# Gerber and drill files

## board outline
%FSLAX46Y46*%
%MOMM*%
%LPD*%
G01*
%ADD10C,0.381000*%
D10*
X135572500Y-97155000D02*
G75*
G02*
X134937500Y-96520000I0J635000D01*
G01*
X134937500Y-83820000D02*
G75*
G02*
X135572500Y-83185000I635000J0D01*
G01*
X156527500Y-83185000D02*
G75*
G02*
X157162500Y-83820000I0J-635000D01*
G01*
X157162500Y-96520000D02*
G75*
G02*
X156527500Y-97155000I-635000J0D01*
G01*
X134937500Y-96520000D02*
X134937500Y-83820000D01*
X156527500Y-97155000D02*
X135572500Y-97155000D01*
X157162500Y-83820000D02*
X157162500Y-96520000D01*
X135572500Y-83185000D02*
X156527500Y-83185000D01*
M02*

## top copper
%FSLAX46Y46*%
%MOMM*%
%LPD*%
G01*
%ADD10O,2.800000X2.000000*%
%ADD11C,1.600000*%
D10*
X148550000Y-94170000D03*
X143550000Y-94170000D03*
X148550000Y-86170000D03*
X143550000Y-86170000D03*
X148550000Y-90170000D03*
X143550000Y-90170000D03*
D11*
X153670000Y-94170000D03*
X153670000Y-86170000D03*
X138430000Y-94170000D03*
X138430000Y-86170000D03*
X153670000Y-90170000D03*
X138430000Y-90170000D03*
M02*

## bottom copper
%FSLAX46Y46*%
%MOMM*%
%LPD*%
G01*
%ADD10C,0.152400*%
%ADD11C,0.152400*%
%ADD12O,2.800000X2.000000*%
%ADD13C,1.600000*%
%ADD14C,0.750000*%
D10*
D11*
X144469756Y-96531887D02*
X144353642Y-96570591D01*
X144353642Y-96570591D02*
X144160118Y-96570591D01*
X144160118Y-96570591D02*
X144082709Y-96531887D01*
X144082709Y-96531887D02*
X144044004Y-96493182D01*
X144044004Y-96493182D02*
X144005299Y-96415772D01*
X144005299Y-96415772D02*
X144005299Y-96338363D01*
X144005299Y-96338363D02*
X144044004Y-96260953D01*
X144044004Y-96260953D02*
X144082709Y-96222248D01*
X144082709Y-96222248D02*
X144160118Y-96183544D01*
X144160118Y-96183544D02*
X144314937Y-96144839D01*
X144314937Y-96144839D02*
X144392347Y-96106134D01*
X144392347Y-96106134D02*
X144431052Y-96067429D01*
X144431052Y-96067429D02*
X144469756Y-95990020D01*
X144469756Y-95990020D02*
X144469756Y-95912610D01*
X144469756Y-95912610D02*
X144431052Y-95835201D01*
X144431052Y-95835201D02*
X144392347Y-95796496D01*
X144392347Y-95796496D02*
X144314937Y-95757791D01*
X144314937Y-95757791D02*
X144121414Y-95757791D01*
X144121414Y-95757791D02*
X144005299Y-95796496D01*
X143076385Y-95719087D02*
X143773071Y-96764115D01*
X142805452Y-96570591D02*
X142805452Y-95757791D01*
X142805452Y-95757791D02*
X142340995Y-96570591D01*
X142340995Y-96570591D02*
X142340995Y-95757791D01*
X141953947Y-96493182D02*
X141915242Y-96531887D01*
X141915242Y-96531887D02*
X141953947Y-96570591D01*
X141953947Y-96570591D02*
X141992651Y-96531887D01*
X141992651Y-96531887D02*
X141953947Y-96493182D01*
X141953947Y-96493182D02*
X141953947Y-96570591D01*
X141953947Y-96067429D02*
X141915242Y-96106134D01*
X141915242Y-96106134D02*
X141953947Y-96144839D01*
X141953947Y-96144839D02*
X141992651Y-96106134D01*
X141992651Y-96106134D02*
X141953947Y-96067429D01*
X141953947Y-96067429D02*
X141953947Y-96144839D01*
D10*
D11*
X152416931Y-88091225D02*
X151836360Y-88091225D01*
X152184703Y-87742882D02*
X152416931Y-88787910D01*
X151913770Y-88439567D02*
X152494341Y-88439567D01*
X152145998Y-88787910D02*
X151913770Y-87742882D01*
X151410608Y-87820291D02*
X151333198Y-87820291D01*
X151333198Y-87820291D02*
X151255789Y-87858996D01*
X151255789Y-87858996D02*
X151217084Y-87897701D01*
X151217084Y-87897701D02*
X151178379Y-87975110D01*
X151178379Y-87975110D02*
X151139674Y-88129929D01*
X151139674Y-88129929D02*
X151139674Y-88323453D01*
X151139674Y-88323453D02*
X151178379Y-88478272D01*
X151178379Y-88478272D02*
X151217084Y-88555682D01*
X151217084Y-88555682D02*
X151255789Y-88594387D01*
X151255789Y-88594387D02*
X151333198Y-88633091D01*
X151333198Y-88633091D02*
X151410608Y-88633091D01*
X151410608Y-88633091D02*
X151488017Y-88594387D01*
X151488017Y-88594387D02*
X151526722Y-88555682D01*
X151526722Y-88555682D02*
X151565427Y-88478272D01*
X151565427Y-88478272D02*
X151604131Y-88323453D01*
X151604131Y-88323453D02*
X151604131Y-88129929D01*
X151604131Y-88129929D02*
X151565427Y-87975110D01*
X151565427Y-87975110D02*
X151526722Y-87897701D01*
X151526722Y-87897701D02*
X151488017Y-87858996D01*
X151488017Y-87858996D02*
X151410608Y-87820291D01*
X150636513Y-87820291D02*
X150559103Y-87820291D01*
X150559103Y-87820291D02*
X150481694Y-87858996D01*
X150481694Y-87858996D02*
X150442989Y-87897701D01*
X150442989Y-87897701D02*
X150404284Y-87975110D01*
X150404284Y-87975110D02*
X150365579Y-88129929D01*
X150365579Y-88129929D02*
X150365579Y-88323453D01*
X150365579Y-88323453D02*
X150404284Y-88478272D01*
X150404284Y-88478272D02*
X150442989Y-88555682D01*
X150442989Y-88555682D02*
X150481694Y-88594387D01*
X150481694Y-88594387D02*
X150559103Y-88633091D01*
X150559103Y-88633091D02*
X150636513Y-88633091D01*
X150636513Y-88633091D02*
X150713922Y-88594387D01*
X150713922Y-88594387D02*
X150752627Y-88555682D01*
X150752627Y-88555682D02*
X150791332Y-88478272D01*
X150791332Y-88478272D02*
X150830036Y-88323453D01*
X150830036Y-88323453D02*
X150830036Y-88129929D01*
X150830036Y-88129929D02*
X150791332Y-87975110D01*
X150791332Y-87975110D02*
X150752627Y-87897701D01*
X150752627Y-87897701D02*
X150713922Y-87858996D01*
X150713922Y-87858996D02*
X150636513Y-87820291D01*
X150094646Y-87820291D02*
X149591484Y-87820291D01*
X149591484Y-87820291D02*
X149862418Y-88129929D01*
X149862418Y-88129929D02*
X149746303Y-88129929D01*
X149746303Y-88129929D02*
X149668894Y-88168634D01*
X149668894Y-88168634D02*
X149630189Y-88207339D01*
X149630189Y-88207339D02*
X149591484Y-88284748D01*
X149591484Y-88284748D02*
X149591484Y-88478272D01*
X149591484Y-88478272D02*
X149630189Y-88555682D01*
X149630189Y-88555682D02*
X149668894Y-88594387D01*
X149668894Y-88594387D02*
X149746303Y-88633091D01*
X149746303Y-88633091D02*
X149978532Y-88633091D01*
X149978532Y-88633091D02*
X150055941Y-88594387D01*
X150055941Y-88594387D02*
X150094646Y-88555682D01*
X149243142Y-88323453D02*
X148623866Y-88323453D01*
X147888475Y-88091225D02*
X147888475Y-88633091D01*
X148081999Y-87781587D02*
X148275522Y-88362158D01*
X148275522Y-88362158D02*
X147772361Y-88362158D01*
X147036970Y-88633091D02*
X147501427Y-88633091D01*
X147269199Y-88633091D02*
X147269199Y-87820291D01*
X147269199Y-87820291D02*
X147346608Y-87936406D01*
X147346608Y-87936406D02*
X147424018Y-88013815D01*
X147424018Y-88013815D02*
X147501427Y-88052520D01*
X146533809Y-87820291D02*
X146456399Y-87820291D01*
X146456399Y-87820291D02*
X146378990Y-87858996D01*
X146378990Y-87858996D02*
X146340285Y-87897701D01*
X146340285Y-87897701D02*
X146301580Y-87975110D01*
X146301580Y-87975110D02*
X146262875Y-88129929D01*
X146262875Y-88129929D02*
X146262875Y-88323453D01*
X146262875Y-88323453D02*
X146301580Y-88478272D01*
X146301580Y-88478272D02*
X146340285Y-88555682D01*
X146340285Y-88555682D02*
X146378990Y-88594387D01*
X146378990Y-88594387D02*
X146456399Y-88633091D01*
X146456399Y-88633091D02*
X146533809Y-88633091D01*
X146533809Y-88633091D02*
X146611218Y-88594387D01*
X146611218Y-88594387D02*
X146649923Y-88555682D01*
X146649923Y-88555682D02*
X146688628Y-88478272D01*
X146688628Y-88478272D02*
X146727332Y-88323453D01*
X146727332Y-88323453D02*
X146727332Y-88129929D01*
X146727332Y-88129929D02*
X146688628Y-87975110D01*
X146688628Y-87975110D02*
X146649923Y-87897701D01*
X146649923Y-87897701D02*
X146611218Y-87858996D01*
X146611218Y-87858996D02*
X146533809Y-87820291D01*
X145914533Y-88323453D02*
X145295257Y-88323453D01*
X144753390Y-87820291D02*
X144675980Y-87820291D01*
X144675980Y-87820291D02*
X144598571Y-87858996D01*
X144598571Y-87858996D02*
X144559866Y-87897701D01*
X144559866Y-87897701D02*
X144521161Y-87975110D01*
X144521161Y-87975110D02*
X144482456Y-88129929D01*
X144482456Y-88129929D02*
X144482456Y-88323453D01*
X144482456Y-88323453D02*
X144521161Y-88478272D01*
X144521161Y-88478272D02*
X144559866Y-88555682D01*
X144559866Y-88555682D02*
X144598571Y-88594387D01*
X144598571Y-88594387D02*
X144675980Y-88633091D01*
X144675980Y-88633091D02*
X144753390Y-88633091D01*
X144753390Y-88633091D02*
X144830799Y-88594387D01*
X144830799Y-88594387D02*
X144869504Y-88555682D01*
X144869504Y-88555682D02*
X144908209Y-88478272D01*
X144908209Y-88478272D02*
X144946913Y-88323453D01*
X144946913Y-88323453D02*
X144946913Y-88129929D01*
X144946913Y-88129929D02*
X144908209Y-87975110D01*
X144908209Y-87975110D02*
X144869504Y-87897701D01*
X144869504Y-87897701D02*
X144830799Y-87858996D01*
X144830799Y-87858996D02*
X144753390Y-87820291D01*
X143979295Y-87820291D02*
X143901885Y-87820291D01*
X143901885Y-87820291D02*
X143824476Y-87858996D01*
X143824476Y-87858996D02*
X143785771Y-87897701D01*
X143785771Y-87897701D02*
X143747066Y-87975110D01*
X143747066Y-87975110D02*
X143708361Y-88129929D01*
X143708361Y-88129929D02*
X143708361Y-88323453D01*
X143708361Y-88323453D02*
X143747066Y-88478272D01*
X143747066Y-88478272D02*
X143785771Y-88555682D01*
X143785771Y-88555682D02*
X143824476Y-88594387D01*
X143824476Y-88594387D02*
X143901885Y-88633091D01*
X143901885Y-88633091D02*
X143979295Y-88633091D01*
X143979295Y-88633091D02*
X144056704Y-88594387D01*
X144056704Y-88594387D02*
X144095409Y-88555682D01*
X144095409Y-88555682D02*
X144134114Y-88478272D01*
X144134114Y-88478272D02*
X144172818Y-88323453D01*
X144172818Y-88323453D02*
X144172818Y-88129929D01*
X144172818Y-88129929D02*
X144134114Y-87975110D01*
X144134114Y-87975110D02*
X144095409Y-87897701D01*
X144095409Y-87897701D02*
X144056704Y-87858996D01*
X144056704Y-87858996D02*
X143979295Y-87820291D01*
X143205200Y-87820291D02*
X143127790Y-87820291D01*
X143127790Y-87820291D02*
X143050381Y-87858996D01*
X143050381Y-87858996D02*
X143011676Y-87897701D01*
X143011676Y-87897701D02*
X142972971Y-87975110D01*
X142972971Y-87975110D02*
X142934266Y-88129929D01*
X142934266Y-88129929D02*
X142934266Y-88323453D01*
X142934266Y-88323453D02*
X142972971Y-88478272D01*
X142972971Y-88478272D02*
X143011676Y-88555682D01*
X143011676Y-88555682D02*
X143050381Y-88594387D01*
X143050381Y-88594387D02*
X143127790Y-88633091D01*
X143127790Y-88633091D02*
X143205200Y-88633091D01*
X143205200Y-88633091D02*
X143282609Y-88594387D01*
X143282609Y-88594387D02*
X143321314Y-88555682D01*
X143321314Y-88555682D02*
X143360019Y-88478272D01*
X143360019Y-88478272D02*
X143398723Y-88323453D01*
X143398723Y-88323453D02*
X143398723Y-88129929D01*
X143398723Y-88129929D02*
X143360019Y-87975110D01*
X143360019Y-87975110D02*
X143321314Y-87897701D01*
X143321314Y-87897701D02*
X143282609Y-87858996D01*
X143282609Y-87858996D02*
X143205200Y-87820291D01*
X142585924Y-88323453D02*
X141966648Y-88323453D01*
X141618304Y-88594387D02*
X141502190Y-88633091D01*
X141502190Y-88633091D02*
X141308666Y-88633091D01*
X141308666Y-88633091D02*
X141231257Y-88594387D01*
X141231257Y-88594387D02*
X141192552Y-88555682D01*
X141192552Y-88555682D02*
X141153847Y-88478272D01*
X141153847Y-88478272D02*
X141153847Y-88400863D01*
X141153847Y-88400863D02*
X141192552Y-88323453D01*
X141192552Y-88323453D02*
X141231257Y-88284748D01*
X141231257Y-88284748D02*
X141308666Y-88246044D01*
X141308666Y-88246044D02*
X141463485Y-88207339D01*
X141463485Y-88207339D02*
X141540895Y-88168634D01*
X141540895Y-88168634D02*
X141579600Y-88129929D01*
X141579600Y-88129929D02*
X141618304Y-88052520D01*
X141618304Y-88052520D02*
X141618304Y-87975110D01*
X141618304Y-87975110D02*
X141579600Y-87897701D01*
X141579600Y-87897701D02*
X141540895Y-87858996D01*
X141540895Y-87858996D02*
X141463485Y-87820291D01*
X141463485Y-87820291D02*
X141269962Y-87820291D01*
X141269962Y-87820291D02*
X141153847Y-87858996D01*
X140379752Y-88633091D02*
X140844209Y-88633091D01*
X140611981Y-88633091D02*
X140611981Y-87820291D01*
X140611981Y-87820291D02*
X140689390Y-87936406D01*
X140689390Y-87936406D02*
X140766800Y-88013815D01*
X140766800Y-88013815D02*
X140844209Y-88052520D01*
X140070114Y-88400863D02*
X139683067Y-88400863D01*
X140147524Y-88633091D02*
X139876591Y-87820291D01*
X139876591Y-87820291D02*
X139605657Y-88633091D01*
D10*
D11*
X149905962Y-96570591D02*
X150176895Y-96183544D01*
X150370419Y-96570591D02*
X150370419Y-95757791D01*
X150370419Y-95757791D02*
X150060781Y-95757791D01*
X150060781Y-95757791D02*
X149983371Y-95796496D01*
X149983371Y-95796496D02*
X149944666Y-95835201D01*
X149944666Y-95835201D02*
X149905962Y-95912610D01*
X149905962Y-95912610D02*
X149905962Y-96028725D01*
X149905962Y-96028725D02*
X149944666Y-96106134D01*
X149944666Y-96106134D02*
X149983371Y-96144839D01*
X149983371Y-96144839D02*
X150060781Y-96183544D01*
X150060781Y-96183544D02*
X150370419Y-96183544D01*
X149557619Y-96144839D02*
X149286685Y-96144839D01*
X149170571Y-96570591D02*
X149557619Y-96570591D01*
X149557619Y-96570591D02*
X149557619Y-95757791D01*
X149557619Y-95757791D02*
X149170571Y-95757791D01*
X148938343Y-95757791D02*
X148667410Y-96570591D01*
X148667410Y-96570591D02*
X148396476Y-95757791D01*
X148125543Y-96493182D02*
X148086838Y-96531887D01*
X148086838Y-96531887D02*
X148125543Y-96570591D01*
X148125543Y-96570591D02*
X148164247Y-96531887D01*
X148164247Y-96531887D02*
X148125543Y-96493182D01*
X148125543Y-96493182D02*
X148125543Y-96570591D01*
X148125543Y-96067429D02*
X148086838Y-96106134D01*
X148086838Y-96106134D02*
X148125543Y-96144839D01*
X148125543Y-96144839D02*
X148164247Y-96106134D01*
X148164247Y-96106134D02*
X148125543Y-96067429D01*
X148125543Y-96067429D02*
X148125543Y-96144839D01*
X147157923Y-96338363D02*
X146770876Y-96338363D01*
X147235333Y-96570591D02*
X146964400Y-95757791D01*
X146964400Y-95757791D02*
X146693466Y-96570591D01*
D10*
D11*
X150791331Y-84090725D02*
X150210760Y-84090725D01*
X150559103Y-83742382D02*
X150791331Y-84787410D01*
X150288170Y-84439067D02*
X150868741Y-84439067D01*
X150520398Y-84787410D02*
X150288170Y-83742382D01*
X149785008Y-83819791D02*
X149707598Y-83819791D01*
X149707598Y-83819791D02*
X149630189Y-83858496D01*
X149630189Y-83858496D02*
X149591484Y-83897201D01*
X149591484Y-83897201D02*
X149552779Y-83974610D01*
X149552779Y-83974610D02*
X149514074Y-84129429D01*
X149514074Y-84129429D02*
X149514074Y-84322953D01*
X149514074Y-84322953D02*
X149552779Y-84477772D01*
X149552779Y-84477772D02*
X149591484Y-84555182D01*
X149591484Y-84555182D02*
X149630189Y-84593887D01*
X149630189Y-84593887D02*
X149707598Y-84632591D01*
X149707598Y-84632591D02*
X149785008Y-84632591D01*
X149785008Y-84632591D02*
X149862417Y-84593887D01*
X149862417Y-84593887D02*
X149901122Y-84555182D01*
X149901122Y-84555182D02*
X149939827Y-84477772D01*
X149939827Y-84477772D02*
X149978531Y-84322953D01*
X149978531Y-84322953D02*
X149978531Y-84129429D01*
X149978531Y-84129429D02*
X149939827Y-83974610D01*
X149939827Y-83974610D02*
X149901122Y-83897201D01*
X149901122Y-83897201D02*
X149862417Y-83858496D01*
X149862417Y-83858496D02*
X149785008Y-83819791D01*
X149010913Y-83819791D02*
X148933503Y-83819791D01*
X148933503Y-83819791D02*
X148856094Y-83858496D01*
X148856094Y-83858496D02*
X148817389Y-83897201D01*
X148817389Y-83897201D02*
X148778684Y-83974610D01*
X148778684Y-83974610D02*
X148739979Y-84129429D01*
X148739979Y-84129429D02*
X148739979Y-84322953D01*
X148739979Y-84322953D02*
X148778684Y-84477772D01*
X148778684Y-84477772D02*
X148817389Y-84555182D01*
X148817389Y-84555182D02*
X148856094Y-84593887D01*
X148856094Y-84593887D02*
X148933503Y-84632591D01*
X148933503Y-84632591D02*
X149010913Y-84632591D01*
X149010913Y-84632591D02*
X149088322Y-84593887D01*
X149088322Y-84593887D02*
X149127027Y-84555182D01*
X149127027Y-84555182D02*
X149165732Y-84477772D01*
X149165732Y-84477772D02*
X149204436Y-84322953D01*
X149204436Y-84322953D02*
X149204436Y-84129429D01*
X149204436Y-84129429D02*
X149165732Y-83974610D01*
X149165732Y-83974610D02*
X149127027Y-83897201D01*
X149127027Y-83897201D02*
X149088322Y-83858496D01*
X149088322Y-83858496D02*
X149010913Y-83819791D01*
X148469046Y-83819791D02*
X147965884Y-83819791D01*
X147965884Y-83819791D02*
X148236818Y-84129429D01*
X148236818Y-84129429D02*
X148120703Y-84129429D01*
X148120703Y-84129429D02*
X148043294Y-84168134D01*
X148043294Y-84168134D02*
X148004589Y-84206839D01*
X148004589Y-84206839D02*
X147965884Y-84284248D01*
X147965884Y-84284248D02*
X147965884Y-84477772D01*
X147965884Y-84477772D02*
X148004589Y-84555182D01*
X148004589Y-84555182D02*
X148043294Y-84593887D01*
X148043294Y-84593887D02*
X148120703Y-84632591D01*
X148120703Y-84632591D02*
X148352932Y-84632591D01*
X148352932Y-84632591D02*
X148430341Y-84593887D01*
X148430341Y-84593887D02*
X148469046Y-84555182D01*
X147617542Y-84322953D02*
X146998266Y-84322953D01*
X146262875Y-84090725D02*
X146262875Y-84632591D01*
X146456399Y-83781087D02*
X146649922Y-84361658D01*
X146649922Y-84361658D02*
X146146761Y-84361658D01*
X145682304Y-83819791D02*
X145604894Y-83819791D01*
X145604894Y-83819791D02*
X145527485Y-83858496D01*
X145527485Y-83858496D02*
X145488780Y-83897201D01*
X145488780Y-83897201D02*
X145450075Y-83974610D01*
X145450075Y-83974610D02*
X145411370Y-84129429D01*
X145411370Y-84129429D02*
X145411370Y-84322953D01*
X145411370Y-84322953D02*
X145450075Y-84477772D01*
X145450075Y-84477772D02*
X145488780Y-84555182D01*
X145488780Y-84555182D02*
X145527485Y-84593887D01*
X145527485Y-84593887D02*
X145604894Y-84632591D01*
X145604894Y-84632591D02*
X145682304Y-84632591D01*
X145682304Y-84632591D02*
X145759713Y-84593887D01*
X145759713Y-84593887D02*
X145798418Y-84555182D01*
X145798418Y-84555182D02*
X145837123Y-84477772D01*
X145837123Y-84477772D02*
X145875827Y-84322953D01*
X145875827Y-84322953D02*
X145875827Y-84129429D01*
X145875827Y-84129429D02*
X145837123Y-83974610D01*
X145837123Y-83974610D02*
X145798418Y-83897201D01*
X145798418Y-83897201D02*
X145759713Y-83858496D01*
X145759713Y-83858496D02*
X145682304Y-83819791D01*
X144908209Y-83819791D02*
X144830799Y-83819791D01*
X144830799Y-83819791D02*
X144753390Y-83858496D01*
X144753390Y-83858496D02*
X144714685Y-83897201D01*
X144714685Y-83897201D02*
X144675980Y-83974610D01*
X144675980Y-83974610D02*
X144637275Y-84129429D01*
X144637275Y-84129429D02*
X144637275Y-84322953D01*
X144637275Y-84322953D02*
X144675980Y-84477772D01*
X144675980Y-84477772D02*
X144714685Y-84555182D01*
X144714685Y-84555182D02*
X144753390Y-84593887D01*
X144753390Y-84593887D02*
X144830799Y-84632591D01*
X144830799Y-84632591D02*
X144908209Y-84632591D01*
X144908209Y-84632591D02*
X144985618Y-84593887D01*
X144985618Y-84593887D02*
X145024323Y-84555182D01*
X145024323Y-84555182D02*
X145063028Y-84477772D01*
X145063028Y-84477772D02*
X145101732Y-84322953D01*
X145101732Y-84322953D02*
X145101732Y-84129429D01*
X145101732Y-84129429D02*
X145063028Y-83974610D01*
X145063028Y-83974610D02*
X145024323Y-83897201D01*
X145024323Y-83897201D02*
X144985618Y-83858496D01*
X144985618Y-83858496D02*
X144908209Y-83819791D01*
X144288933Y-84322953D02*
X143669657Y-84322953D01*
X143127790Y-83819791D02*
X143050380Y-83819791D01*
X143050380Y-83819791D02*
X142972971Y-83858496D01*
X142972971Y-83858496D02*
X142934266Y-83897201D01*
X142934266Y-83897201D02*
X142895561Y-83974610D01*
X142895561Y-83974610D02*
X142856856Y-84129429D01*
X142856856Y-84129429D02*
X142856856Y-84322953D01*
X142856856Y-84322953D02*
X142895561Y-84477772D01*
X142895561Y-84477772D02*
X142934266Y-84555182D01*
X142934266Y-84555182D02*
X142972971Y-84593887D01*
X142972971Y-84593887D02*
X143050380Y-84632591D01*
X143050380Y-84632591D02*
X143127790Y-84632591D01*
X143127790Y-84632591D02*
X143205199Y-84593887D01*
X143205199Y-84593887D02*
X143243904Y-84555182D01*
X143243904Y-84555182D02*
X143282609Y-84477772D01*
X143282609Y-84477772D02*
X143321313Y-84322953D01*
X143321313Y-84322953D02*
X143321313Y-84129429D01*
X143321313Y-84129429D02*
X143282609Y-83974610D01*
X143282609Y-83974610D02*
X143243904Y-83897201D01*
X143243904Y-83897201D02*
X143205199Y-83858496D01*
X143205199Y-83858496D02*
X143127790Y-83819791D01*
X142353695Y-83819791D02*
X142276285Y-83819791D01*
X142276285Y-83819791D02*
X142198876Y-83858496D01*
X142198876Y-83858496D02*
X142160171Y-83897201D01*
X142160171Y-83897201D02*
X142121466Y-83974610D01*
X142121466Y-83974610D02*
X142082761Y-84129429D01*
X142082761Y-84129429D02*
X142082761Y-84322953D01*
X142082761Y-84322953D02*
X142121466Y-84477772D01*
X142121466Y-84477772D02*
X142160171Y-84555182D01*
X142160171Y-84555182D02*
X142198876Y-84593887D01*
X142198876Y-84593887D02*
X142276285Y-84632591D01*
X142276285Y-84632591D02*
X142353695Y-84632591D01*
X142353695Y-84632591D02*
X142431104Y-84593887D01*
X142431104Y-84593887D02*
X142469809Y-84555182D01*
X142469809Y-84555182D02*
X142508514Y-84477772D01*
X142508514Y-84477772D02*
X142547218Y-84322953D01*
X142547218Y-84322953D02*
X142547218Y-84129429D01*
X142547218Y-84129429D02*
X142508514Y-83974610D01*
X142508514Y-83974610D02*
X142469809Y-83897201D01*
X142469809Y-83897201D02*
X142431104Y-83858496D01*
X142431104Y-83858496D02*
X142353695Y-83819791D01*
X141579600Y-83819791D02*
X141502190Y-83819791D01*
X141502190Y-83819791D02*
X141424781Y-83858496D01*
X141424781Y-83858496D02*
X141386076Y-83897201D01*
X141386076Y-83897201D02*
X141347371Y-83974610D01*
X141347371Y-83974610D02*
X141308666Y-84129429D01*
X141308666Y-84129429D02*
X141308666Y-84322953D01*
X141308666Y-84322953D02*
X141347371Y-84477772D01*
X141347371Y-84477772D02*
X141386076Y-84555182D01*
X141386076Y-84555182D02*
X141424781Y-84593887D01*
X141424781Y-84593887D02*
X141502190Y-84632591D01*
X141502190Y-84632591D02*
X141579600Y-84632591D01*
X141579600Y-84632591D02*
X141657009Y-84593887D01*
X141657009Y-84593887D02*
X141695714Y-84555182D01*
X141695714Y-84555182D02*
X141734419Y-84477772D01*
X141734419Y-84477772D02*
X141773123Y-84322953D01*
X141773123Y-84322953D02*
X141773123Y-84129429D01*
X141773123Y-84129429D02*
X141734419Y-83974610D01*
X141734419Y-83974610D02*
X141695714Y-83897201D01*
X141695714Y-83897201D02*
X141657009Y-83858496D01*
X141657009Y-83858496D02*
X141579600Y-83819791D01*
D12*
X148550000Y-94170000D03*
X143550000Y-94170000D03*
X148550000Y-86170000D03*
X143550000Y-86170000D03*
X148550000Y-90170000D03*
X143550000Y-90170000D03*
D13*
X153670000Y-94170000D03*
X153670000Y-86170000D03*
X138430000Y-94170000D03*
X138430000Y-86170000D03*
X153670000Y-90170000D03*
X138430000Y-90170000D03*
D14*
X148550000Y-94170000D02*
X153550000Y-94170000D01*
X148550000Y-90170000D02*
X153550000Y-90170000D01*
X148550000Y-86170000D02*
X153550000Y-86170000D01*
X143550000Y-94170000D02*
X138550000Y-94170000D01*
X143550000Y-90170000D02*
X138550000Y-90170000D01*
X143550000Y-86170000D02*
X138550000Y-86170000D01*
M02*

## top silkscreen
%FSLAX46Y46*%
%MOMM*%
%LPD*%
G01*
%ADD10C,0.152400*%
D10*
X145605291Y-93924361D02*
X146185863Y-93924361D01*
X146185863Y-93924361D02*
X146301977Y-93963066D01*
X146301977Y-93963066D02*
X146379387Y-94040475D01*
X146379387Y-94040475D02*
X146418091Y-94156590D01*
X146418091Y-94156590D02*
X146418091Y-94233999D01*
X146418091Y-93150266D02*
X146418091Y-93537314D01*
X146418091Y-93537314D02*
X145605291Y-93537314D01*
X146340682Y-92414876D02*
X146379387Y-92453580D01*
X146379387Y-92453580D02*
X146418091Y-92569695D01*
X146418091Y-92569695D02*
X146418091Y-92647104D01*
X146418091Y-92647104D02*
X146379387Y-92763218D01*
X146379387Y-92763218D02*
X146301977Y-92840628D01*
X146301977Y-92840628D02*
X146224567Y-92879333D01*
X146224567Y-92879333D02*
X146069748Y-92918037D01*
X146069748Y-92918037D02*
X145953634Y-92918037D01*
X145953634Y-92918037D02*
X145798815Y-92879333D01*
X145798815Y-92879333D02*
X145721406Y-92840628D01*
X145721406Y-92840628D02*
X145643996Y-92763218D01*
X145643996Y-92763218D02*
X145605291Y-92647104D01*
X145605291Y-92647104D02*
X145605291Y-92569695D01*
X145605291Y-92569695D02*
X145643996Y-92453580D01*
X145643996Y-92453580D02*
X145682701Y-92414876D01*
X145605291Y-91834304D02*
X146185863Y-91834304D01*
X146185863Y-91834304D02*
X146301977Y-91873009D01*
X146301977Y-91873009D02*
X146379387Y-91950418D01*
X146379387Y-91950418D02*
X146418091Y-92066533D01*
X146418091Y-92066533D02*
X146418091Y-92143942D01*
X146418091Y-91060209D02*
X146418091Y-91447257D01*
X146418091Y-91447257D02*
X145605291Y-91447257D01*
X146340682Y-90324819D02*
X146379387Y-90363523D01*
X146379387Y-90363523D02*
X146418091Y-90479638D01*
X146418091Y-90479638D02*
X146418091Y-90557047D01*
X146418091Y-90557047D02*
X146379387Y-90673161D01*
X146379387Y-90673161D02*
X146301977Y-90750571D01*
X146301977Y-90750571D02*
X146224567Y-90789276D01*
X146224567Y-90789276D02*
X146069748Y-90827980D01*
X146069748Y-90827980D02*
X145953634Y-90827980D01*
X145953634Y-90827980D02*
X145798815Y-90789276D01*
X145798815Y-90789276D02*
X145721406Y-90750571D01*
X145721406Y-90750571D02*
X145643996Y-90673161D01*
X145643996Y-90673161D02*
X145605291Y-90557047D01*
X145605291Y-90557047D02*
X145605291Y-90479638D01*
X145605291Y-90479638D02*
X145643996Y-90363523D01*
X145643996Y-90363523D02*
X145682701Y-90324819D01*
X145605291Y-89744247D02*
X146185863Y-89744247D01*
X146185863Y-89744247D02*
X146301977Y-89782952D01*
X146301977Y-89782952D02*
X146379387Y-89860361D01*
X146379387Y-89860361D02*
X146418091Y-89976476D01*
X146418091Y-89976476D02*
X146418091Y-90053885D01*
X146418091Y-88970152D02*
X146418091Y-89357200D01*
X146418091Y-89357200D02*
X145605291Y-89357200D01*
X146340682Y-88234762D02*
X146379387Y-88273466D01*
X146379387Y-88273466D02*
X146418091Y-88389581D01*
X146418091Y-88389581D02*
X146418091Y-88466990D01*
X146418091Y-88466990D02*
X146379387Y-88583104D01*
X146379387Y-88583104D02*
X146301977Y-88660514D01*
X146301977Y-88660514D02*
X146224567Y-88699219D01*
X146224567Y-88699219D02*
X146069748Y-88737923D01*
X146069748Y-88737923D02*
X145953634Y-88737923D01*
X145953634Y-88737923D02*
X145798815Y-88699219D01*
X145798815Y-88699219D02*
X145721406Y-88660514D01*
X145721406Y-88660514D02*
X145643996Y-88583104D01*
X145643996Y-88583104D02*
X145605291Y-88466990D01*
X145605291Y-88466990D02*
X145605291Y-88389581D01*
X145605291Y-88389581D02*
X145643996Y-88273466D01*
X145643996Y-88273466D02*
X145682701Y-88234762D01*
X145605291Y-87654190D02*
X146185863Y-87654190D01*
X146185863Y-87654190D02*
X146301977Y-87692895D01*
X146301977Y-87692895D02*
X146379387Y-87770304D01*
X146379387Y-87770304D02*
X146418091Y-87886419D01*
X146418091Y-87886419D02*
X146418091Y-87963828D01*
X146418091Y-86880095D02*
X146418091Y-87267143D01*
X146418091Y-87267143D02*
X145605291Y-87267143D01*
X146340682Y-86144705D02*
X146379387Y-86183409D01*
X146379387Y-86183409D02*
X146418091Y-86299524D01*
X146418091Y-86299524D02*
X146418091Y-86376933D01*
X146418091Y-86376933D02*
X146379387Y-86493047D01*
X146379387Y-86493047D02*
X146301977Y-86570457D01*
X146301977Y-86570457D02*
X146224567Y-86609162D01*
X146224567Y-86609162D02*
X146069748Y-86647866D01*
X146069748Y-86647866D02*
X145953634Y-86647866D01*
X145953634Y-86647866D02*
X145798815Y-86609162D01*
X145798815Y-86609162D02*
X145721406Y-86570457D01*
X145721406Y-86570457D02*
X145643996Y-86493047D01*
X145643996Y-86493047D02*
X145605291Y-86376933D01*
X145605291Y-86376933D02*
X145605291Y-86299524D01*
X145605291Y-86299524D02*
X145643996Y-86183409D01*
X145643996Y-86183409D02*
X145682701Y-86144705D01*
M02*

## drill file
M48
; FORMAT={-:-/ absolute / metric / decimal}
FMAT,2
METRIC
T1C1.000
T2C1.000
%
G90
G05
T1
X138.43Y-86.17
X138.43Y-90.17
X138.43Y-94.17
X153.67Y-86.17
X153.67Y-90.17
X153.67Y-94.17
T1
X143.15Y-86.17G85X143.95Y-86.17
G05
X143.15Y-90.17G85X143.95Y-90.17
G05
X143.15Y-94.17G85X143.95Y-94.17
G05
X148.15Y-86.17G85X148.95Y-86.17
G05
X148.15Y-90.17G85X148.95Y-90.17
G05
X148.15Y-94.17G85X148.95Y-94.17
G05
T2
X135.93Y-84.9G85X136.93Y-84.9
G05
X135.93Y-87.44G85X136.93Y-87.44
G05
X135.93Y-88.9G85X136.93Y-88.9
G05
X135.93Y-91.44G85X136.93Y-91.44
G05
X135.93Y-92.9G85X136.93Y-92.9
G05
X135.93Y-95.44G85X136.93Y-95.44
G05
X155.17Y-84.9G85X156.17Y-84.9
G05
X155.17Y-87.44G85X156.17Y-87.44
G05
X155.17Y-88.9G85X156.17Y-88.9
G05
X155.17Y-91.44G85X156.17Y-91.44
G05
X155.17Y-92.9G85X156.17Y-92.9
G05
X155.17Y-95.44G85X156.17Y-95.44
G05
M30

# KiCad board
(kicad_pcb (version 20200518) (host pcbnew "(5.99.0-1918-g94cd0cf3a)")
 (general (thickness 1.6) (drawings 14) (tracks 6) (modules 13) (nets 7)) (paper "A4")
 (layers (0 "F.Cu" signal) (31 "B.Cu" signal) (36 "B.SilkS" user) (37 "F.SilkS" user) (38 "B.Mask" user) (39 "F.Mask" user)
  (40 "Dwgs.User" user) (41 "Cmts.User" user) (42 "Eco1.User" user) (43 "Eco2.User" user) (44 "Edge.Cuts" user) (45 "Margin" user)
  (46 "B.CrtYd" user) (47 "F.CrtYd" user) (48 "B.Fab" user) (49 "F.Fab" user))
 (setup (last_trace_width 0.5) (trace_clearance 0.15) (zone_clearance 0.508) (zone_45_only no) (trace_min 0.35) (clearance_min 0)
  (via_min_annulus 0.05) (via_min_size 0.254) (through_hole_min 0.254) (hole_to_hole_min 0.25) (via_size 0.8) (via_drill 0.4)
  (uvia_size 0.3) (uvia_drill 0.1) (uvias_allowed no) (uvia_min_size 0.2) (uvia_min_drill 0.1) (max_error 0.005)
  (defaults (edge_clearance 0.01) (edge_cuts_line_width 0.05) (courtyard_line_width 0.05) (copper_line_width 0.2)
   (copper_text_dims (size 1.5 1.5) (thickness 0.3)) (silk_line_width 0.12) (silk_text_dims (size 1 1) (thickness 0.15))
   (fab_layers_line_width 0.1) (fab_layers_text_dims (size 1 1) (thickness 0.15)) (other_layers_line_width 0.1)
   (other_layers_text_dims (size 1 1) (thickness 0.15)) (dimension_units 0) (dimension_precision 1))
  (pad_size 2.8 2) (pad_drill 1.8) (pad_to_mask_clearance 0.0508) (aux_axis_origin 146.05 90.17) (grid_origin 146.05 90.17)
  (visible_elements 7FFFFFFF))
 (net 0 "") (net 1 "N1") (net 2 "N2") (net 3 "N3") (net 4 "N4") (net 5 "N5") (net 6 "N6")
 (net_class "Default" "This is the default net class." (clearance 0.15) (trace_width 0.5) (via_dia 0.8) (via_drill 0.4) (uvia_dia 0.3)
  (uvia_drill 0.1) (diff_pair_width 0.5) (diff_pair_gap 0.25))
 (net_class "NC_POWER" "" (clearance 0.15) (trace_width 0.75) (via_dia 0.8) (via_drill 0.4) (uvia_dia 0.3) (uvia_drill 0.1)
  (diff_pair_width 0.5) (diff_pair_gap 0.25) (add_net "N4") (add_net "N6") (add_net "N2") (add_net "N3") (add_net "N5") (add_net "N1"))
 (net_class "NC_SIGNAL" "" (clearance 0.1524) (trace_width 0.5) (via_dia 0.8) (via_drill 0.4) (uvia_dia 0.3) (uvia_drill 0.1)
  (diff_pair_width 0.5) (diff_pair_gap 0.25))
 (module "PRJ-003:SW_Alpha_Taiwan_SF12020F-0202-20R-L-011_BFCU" (layer "F.Cu") (at 146.05 90.17)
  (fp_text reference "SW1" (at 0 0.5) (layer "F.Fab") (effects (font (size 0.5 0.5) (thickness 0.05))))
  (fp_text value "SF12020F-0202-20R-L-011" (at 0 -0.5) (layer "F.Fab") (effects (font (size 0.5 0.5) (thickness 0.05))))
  (pad "" connect oval (at 2.5 4) (size 1.8 1) (layers "F.Mask"))
  (pad "6" thru_hole oval (at 2.5 4) (size 2.8 2) (drill oval 1.8 1) (layers *.Cu *.Mask) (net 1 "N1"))
  (pad "3" thru_hole oval (at -2.5 4) (size 2.8 2) (drill oval 1.8 1) (layers *.Cu *.Mask) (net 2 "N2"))
  (pad "4" thru_hole oval (at 2.5 -4) (size 2.8 2) (drill oval 1.8 1) (layers *.Cu *.Mask) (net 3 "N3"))
  (pad "1" thru_hole oval (at -2.5 -4) (size 2.8 2) (drill oval 1.8 1) (layers *.Cu *.Mask) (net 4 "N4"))
  (pad "5" thru_hole oval (at 2.5 0) (size 2.8 2) (drill oval 1.8 1) (layers *.Cu *.Mask) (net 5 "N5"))
  (pad "2" thru_hole oval (at -2.5 0) (size 2.8 2) (drill oval 1.8 1) (layers *.Cu *.Mask) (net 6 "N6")))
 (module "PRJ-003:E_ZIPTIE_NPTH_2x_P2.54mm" (layer "F.Cu") (at 155.67 94.17 90)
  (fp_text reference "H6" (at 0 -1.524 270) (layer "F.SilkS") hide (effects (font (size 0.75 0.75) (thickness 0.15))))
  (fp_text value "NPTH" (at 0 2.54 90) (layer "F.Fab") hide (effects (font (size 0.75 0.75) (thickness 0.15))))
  (pad "" np_thru_hole oval (at 1.27 0 90) (size 1 2) (drill oval 1 2) (layers *.Cu *.Mask))
  (pad "" np_thru_hole oval (at -1.27 0 90) (size 1 2) (drill oval 1 2) (layers *.Cu *.Mask)))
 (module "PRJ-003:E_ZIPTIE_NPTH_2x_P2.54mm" (layer "F.Cu") (at 155.67 90.17 90)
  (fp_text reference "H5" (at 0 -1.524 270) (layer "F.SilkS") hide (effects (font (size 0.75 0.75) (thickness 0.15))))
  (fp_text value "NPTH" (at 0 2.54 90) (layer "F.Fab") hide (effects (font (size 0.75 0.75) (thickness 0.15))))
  (pad "" np_thru_hole oval (at 1.27 0 90) (size 1 2) (drill oval 1 2) (layers *.Cu *.Mask))
  (pad "" np_thru_hole oval (at -1.27 0 90) (size 1 2) (drill oval 1 2) (layers *.Cu *.Mask)))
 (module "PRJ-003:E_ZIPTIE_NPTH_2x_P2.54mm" (layer "F.Cu") (at 155.67 86.17 90)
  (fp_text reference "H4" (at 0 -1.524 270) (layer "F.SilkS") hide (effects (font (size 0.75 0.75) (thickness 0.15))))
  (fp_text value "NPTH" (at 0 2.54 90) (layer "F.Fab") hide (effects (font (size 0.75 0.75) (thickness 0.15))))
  (pad "" np_thru_hole oval (at 1.27 0 90) (size 1 2) (drill oval 1 2) (layers *.Cu *.Mask))
  (pad "" np_thru_hole oval (at -1.27 0 90) (size 1 2) (drill oval 1 2) (layers *.Cu *.Mask)))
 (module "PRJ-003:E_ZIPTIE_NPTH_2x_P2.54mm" (layer "F.Cu") (at 136.43 94.17 90)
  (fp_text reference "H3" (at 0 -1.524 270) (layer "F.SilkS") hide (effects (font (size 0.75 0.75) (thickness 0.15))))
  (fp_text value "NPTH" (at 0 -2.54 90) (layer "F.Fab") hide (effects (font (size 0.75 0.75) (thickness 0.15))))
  (pad "" np_thru_hole oval (at 1.27 0 90) (size 1 2) (drill oval 1 2) (layers *.Cu *.Mask))
  (pad "" np_thru_hole oval (at -1.27 0 90) (size 1 2) (drill oval 1 2) (layers *.Cu *.Mask)))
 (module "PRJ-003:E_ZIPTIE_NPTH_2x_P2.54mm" (layer "F.Cu") (at 136.43 90.17 90)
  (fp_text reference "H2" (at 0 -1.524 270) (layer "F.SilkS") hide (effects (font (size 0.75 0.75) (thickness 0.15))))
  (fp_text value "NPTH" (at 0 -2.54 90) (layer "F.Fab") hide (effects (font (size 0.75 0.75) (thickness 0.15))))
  (pad "" np_thru_hole oval (at 1.27 0 90) (size 1 2) (drill oval 1 2) (layers *.Cu *.Mask))
  (pad "" np_thru_hole oval (at -1.27 0 90) (size 1 2) (drill oval 1 2) (layers *.Cu *.Mask)))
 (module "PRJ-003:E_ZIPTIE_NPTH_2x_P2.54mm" (layer "F.Cu") (at 136.43 86.17 90)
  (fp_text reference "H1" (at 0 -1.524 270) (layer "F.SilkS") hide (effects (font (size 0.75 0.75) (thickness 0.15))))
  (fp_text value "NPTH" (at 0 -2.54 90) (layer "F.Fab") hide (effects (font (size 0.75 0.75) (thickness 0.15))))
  (pad "" np_thru_hole oval (at 1.27 0 90) (size 1 2) (drill oval 1 2) (layers *.Cu *.Mask))
  (pad "" np_thru_hole oval (at -1.27 0 90) (size 1 2) (drill oval 1 2) (layers *.Cu *.Mask)))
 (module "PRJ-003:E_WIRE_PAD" (layer "F.Cu") (at 153.67 94.17)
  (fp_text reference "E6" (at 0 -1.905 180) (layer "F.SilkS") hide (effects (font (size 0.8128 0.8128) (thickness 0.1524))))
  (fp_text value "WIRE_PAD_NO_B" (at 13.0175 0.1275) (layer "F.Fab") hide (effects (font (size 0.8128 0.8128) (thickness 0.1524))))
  (pad "" connect circle (at 0 0) (size 1 1) (layers "F.Mask"))
  (pad "1" thru_hole circle (at 0 0) (size 1.6 1.6) (drill 1) (layers "B.Cu" "B.Mask") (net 1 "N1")))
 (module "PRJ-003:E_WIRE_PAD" (layer "F.Cu") (at 153.67 86.17)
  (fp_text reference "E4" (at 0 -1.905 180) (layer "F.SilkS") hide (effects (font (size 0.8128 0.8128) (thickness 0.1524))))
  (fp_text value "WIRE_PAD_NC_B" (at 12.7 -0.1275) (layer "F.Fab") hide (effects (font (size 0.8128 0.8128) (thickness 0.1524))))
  (pad "" connect circle (at 0 0) (size 1 1) (layers "F.Mask"))
  (pad "1" thru_hole circle (at 0 0) (size 1.6 1.6) (drill 1) (layers "B.Cu" "B.Mask") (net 3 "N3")))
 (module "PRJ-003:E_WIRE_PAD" (layer "F.Cu") (at 138.43 94.17)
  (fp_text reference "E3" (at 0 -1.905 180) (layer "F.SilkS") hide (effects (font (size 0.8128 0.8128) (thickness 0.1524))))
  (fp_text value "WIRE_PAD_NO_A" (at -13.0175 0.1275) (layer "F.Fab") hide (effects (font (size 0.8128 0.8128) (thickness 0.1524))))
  (pad "" connect circle (at 0 0) (size 1 1) (layers "F.Mask"))
  (pad "1" thru_hole circle (at 0 0) (size 1.6 1.6) (drill 1) (layers "B.Cu" "B.Mask") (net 2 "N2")))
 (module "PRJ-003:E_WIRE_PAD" (layer "F.Cu") (at 138.43 86.17)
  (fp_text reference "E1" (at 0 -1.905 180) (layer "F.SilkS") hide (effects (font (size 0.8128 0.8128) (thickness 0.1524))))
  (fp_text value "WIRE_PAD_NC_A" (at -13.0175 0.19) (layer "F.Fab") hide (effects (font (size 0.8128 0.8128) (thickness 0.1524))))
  (pad "" connect circle (at 0 0) (size 1 1) (layers "F.Mask"))
  (pad "1" thru_hole circle (at 0 0) (size 1.6 1.6) (drill 1) (layers "B.Cu" "B.Mask") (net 4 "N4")))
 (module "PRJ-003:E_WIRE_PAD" (layer "F.Cu") (at 153.67 90.17)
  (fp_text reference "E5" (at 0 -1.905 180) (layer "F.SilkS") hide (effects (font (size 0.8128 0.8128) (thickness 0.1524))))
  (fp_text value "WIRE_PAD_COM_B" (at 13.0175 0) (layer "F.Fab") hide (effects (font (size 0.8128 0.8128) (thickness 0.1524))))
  (pad "" connect circle (at 0 0) (size 1 1) (layers "F.Mask"))
  (pad "1" thru_hole circle (at 0 0) (size 1.6 1.6) (drill 1) (layers "B.Cu" "B.Mask") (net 5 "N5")))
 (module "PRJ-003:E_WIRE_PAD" (layer "F.Cu") (at 138.43 90.17)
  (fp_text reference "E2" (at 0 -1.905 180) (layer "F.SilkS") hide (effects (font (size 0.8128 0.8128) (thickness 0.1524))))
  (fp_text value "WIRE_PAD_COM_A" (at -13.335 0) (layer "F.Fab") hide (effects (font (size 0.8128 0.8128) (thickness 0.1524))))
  (pad "" connect circle (at 0 0) (size 1 1) (layers "F.Mask"))
  (pad "1" thru_hole circle (at 0 0) (size 1.6 1.6) (drill 1) (layers "B.Cu" "B.Mask") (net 6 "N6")))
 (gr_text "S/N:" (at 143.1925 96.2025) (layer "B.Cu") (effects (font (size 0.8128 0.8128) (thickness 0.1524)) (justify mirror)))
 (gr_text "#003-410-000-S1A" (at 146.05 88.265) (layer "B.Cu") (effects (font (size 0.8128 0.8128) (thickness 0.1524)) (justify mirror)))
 (gr_arc (start 135.5725 96.52) (end 134.9375 96.52) (angle -90) (layer "Edge.Cuts") (width 0.381))
 (gr_arc (start 135.5725 83.82) (end 135.5725 83.185) (angle -90) (layer "Edge.Cuts") (width 0.381))
 (gr_arc (start 156.5275 83.82) (end 157.1625 83.82) (angle -90) (layer "Edge.Cuts") (width 0.381))
 (gr_arc (start 156.5275 96.52) (end 156.5275 97.155) (angle -90) (layer "Edge.Cuts") (width 0.381))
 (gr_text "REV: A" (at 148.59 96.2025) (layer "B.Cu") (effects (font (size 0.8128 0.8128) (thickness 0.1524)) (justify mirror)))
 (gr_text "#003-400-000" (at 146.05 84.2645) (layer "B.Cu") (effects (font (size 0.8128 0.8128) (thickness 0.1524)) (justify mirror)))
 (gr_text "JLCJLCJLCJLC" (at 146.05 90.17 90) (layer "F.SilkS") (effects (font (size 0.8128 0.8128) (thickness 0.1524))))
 (gr_line (start 134.9375 96.52) (end 134.9375 83.82) (layer "Edge.Cuts") (width 0.381))
 (gr_line (start 156.5275 97.155) (end 135.5725 97.155) (layer "Edge.Cuts") (width 0.381))
 (gr_line (start 157.1625 83.82) (end 157.1625 96.52) (layer "Edge.Cuts") (width 0.381))
 (gr_line (start 135.5725 83.185) (end 156.5275 83.185) (layer "Edge.Cuts") (width 0.381))
 (segment (start 148.55 94.17) (end 153.55 94.17) (width 0.75) (layer "B.Cu") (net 1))
 (segment (start 148.55 90.17) (end 153.55 90.17) (width 0.75) (layer "B.Cu") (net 5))
 (segment (start 148.55 86.17) (end 153.55 86.17) (width 0.75) (layer "B.Cu") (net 3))
 (segment (start 143.55 94.17) (end 138.55 94.17) (width 0.75) (layer "B.Cu") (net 2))
 (segment (start 143.55 90.17) (end 138.55 90.17) (width 0.75) (layer "B.Cu") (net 6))
 (segment (start 143.55 86.17) (end 138.55 86.17) (width 0.75) (layer "B.Cu") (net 4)))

